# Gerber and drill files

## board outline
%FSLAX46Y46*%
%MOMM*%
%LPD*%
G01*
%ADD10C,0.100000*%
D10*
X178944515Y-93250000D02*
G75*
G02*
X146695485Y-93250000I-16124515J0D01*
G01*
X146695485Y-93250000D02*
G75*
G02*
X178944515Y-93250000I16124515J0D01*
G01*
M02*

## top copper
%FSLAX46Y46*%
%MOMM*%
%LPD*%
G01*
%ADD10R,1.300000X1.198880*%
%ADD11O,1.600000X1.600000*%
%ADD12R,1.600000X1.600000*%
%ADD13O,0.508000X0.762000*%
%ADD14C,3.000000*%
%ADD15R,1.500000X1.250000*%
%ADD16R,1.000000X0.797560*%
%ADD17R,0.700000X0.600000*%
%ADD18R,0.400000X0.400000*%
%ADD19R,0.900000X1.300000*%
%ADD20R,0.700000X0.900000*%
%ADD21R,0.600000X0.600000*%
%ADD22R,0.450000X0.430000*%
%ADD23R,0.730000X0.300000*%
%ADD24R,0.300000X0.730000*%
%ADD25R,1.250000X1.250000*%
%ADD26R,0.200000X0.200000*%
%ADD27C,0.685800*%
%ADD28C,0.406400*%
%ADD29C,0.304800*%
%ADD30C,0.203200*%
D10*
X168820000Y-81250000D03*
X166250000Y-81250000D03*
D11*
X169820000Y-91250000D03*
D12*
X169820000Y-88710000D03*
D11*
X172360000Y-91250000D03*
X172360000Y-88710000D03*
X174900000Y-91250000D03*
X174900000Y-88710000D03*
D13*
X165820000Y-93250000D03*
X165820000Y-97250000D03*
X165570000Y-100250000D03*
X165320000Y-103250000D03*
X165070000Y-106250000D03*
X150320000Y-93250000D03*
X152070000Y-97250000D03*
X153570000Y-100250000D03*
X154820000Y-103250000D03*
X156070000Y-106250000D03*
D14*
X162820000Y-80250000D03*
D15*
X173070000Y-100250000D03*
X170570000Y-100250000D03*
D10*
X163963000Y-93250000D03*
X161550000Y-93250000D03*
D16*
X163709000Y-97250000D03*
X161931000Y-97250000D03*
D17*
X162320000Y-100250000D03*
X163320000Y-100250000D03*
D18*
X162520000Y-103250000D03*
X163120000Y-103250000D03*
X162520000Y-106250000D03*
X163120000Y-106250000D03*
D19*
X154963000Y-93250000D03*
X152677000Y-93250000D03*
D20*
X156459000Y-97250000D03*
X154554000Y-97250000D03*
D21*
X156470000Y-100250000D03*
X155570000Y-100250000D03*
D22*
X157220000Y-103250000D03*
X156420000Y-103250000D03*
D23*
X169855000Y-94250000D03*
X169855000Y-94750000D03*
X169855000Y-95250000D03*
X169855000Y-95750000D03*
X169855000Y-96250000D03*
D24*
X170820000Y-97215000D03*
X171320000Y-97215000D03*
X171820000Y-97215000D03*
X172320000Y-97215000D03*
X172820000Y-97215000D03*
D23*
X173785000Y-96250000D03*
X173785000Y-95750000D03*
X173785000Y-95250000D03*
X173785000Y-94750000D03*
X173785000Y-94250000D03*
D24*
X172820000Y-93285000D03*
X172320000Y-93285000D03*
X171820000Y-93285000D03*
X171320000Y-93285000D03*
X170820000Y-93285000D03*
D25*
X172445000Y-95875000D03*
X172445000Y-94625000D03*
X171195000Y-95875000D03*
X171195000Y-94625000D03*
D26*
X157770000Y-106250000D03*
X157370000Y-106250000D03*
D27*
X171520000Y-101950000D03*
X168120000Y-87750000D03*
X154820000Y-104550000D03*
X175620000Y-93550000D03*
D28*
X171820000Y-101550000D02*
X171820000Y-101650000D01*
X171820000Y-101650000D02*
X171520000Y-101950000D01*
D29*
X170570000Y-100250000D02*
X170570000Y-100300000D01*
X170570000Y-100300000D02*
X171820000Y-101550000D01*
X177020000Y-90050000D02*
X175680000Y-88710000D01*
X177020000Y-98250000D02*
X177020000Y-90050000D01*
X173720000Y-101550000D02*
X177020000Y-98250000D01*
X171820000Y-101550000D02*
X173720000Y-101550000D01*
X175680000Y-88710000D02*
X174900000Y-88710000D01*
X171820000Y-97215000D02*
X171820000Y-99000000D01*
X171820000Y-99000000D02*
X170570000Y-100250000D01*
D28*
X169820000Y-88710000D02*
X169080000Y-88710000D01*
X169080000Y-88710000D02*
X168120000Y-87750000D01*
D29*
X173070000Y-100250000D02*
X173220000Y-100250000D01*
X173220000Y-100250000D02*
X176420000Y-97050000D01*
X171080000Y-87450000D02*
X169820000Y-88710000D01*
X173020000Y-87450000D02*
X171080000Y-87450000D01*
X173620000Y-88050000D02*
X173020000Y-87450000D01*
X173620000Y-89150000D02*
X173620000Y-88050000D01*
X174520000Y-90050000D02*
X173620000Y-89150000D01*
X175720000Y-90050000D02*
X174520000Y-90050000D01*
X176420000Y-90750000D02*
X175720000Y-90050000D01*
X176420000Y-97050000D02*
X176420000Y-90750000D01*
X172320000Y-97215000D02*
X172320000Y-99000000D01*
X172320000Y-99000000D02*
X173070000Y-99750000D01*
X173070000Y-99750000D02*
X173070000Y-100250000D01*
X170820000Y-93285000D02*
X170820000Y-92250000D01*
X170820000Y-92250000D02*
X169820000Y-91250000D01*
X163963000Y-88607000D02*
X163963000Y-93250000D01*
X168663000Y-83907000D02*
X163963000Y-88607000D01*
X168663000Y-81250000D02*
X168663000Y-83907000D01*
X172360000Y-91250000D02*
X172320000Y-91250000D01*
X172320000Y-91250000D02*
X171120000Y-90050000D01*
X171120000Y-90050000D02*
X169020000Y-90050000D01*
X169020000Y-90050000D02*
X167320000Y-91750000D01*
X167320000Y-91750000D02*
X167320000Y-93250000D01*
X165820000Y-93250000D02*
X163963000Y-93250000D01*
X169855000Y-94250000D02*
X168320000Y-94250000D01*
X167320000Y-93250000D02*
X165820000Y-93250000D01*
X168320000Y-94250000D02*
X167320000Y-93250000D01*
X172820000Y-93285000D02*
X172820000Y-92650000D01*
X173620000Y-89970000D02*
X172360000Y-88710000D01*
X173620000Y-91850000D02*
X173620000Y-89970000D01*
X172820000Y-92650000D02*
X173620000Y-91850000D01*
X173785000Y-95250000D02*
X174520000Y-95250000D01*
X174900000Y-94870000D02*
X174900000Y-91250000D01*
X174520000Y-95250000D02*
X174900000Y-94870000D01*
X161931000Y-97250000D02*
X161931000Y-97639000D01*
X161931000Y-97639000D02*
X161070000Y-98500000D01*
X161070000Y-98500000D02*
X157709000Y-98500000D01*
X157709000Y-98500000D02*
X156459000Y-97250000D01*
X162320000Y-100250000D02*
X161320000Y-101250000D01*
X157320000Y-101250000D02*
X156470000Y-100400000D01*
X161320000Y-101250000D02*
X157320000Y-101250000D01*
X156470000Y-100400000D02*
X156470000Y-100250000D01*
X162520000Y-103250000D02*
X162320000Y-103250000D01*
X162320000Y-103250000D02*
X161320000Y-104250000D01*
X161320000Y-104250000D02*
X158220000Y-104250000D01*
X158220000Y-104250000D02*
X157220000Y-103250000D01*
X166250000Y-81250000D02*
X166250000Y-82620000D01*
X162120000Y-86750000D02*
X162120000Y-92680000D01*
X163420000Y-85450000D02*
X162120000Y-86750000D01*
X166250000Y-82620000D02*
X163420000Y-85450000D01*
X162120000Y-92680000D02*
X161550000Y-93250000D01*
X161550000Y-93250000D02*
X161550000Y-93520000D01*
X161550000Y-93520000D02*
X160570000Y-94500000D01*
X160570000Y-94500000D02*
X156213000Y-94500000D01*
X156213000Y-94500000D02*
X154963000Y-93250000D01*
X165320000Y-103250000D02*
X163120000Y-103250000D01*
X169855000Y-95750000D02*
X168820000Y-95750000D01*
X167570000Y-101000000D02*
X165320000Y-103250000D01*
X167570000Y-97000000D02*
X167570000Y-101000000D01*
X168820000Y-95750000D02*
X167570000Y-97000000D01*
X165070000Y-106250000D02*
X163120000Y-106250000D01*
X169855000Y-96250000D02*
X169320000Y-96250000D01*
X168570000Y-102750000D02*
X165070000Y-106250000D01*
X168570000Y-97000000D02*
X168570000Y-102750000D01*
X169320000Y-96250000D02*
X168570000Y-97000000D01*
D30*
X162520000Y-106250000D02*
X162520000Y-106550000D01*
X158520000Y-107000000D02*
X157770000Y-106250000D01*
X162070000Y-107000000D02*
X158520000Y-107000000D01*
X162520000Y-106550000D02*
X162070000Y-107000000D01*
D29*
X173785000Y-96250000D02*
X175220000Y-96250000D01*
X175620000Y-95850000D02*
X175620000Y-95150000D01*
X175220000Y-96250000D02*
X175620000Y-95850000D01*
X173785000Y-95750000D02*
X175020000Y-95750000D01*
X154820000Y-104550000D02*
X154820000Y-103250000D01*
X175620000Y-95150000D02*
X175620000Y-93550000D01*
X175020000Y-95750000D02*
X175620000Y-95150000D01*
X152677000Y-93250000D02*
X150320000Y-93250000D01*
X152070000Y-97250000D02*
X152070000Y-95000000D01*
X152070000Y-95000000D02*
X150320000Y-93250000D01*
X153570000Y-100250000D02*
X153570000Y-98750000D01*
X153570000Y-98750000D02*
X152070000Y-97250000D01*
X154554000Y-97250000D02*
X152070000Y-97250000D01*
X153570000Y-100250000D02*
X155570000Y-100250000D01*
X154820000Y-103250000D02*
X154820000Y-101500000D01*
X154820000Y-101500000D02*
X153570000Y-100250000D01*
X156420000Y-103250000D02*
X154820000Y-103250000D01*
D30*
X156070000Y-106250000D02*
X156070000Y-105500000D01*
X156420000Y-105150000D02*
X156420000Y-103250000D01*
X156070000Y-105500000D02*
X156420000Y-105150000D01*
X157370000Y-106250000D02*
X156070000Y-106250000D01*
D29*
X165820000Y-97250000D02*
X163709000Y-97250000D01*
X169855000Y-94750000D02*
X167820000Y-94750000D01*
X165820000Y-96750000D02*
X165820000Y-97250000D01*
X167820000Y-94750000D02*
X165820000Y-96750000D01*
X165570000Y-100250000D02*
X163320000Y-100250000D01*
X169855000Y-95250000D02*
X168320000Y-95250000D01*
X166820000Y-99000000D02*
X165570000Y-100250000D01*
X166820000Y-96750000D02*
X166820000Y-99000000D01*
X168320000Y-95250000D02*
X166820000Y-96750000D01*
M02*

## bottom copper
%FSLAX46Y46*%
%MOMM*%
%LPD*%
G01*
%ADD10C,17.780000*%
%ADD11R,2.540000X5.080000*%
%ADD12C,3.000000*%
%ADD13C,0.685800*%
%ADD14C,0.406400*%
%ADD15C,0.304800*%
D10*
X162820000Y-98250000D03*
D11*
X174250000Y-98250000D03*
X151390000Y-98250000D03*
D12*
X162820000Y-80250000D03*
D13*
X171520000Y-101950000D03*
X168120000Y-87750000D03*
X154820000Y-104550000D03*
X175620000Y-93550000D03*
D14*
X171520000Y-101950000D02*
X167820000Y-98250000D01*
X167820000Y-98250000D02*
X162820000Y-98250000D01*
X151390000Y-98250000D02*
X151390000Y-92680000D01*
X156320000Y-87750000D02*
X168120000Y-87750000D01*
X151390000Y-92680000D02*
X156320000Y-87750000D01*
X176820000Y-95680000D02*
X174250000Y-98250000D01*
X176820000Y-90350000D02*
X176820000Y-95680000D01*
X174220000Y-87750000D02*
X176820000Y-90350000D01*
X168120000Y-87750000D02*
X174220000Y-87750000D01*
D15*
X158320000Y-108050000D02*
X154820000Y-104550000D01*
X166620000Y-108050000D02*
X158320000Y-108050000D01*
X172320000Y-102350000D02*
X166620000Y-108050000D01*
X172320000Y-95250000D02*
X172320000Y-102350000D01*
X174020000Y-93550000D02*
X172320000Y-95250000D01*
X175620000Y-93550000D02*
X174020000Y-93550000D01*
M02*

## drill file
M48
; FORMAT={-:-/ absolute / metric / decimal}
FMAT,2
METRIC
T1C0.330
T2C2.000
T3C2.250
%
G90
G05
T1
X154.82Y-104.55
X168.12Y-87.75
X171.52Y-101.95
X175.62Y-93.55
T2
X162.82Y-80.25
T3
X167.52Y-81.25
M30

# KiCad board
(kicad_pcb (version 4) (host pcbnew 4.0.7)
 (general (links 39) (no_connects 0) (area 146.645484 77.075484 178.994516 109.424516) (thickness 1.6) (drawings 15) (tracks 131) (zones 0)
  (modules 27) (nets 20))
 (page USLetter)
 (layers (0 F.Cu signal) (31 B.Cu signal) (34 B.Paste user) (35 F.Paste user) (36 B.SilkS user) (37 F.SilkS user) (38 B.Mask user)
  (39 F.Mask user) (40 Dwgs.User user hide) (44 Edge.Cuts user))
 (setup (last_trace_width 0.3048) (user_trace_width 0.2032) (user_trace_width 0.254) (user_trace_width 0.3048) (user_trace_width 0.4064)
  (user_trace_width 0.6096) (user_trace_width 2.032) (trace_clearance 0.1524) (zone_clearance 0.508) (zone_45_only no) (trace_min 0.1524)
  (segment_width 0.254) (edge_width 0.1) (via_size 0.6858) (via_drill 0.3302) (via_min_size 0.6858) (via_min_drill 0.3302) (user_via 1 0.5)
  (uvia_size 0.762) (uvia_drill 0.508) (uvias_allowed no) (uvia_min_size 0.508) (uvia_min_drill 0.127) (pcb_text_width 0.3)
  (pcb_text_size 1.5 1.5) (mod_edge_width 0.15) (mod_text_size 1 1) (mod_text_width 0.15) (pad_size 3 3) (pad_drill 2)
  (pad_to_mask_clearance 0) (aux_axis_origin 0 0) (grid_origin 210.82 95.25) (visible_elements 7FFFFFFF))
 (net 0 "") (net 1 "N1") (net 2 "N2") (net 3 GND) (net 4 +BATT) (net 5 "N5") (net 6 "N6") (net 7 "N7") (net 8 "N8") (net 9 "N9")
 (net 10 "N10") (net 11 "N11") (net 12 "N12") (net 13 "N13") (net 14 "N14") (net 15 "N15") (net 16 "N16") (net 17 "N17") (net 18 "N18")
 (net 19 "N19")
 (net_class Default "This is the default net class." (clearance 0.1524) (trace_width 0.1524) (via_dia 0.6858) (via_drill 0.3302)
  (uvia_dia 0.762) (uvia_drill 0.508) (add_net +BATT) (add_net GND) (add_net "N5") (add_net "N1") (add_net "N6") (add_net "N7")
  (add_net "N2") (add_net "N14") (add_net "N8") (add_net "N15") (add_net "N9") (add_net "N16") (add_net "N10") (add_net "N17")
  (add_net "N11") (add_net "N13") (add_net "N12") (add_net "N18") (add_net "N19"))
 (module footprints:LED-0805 (layer F.Cu) (at 167.52 81.25)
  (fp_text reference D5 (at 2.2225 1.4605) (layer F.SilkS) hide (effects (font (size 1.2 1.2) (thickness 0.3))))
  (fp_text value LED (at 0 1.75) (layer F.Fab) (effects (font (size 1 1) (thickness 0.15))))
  (pad 2 smd rect (at 1.3 0 180) (size 1.3 1.19888) (layers F.Cu F.Paste F.Mask) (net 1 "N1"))
  (pad 1 smd rect (at -1.27 0 180) (size 1.3 1.19888) (layers F.Cu F.Paste F.Mask) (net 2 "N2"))
  (pad "" np_thru_hole circle (at 0 0) (size 2.25 2.25) (drill 2.25) (layers *.Cu *.Mask)))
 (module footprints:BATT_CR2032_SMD (layer B.Cu) (at 162.82 98.25 180)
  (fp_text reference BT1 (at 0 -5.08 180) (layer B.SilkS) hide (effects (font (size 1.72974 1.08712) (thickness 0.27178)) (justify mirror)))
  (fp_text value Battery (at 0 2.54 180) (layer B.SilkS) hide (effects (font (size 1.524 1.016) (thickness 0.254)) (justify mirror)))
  (pad 2 smd circle (at 0 0 180) (size 17.78 17.78) (layers B.Cu B.Paste B.Mask) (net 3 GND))
  (pad 1 smd rect (at -11.43 0 180) (size 2.54 5.08) (layers B.Cu B.Paste B.Mask) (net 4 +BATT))
  (pad 1 smd rect (at 11.43 0 180) (size 2.54 5.08) (layers B.Cu B.Paste B.Mask) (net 4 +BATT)))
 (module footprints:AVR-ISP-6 (layer F.Cu) (at 169.82 91.25 90)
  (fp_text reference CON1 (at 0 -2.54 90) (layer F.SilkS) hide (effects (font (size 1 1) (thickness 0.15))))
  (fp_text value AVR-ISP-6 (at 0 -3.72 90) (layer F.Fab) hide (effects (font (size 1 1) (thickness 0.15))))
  (pad 1 smd oval (at 0 0 90) (size 1.6 1.6) (layers F.Cu F.Paste F.Mask) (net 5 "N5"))
  (pad 2 smd rect (at 2.54 0 90) (size 1.6 1.6) (layers F.Cu F.Paste F.Mask) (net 4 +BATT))
  (pad 3 smd oval (at 0 2.54 90) (size 1.6 1.6) (layers F.Cu F.Paste F.Mask) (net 1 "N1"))
  (pad 4 smd oval (at 2.54 2.54 90) (size 1.6 1.6) (layers F.Cu F.Paste F.Mask) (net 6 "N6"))
  (pad 5 smd oval (at 0 5.08 90) (size 1.6 1.6) (layers F.Cu F.Paste F.Mask) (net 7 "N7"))
  (pad 6 smd oval (at 2.54 5.08 90) (size 1.6 1.6) (layers F.Cu F.Paste F.Mask) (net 3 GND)))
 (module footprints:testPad (layer F.Cu) (at 165.82 93.25)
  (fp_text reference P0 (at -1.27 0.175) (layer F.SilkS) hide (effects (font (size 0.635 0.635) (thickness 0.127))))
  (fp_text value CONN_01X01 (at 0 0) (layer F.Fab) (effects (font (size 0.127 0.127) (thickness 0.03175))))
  (pad 1 smd oval (at 0 0) (size 0.508 0.762) (layers F.Cu F.Paste F.Mask) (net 1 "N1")))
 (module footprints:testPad (layer F.Cu) (at 165.82 97.25)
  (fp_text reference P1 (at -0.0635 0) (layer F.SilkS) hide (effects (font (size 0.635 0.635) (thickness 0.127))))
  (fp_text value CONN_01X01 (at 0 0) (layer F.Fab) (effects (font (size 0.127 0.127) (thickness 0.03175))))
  (pad 1 smd oval (at 0 0) (size 0.508 0.762) (layers F.Cu F.Paste F.Mask) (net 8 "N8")))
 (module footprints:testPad (layer F.Cu) (at 165.57 100.25)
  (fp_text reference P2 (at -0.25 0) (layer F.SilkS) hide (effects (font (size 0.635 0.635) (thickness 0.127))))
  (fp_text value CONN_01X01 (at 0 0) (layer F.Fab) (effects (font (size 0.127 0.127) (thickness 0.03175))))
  (pad 1 smd oval (at 0 0) (size 0.508 0.762) (layers F.Cu F.Paste F.Mask) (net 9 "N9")))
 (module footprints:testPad (layer F.Cu) (at 165.32 103.25)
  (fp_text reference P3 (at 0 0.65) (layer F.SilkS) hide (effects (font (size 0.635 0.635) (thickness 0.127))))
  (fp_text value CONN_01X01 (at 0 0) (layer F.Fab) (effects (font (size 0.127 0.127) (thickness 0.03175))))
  (pad 1 smd oval (at 0 0) (size 0.508 0.762) (layers F.Cu F.Paste F.Mask) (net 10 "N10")))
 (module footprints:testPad (layer F.Cu) (at 165.07 106.25)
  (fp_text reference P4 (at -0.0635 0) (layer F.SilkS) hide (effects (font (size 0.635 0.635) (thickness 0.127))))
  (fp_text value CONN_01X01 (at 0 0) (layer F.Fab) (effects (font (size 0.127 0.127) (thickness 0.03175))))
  (pad 1 smd oval (at 0 0) (size 0.508 0.762) (layers F.Cu F.Paste F.Mask) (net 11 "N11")))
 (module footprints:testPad (layer F.Cu) (at 150.32 93.25)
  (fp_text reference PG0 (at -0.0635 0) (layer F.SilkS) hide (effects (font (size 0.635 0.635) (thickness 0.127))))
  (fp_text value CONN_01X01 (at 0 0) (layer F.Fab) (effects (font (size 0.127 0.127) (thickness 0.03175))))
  (pad 1 smd oval (at 0 0) (size 0.508 0.762) (layers F.Cu F.Paste F.Mask) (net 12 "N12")))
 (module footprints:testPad (layer F.Cu) (at 152.07 97.25)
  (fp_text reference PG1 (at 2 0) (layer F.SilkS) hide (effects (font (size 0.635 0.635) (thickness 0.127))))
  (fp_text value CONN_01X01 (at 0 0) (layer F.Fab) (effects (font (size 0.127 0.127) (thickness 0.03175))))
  (pad 1 smd oval (at 0 0) (size 0.508 0.762) (layers F.Cu F.Paste F.Mask) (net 12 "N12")))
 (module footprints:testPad (layer F.Cu) (at 153.57 100.25)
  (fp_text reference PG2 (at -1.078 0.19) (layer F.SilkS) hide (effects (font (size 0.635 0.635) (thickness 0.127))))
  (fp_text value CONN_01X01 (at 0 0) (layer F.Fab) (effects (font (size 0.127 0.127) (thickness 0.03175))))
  (pad 1 smd oval (at 0 0) (size 0.508 0.762) (layers F.Cu F.Paste F.Mask) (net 12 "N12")))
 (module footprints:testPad (layer F.Cu) (at 154.82 103.25)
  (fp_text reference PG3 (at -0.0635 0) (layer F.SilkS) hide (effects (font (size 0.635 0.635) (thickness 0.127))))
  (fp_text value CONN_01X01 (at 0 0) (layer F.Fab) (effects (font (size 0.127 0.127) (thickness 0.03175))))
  (pad 1 smd oval (at 0 0) (size 0.508 0.762) (layers F.Cu F.Paste F.Mask) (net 12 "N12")))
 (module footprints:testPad (layer F.Cu) (at 156.07 106.25)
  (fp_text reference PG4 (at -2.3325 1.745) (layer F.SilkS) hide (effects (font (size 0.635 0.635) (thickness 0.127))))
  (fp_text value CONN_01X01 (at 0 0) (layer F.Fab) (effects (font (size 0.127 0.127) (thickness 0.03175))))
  (pad 1 smd oval (at 0 0) (size 0.508 0.762) (layers F.Cu F.Paste F.Mask) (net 12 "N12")))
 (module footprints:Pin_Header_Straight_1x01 (layer F.Cu) (at 162.82 80.25)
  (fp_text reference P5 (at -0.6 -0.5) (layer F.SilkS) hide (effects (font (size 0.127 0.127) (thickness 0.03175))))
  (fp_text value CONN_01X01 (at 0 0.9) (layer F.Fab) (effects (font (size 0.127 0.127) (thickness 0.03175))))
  (pad 1 thru_hole circle (at 0 0) (size 3 3) (drill 2) (layers *.Cu *.Mask) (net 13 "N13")))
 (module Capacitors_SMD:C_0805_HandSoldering (layer F.Cu) (at 171.82 100.25 180)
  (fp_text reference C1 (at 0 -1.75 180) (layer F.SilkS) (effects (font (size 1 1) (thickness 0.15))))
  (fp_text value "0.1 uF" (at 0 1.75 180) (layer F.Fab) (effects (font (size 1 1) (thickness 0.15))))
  (pad 1 smd rect (at -1.25 0 180) (size 1.5 1.25) (layers F.Cu F.Paste F.Mask) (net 4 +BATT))
  (pad 2 smd rect (at 1.25 0 180) (size 1.5 1.25) (layers F.Cu F.Paste F.Mask) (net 3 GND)))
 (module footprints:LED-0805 (layer F.Cu) (at 162.82 93.25)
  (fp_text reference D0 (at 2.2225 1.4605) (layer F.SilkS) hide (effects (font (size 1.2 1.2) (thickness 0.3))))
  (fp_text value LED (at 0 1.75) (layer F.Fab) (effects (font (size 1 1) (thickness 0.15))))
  (pad 2 smd rect (at 1.143 0 180) (size 1.3 1.19888) (layers F.Cu F.Paste F.Mask) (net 1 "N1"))
  (pad 1 smd rect (at -1.27 0 180) (size 1.3 1.19888) (layers F.Cu F.Paste F.Mask) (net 2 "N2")))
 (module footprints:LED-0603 (layer F.Cu) (at 162.82 97.25)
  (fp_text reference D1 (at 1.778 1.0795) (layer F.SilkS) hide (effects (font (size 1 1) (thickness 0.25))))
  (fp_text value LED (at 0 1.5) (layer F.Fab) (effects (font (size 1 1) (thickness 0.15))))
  (pad 2 smd rect (at 0.889 0 180) (size 1 0.79756) (layers F.Cu F.Paste F.Mask) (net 8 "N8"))
  (pad 1 smd rect (at -0.889 0 180) (size 1 0.79756) (layers F.Cu F.Paste F.Mask) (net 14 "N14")))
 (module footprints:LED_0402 (layer F.Cu) (at 162.82 100.25)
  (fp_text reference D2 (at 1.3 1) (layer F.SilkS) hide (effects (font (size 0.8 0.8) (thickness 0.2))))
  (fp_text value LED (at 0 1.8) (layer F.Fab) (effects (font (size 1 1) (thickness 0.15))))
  (pad 1 smd rect (at -0.5 0) (size 0.7 0.6) (layers F.Cu F.Paste F.Mask) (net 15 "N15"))
  (pad 2 smd rect (at 0.5 0) (size 0.7 0.6) (layers F.Cu F.Paste F.Mask) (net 9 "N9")))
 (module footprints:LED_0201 (layer F.Cu) (at 162.82 103.25)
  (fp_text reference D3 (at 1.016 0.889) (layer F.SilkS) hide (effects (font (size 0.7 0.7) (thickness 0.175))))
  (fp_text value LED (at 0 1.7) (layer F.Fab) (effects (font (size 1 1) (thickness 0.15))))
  (pad 1 smd rect (at -0.3 0) (size 0.4 0.4) (layers F.Cu F.Paste F.Mask) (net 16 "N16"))
  (pad 2 smd rect (at 0.3 0) (size 0.4 0.4) (layers F.Cu F.Paste F.Mask) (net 10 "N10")))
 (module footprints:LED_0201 (layer F.Cu) (at 162.82 106.25)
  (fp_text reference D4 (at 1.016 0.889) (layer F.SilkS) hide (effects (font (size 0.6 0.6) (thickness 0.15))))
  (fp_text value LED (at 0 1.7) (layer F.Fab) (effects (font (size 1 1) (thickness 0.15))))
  (pad 1 smd rect (at -0.3 0) (size 0.4 0.4) (layers F.Cu F.Paste F.Mask) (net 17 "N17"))
  (pad 2 smd rect (at 0.3 0) (size 0.4 0.4) (layers F.Cu F.Paste F.Mask) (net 11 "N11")))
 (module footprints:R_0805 (layer F.Cu) (at 153.82 93.25 180)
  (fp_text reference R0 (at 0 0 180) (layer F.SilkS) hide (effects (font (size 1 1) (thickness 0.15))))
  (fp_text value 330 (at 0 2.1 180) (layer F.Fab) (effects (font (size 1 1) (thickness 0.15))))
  (pad 1 smd rect (at -1.143 0 180) (size 0.9 1.3) (layers F.Cu F.Paste F.Mask) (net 2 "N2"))
  (pad 2 smd rect (at 1.143 0 180) (size 0.9 1.3) (layers F.Cu F.Paste F.Mask) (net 12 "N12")))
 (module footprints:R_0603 (layer F.Cu) (at 155.57 97.25 180)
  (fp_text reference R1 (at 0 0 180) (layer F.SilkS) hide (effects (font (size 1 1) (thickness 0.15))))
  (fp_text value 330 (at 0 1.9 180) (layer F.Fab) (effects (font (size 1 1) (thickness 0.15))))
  (pad 1 smd rect (at -0.889 0 180) (size 0.7 0.9) (layers F.Cu F.Paste F.Mask) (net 14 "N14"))
  (pad 2 smd rect (at 1.016 0 180) (size 0.7 0.9) (layers F.Cu F.Paste F.Mask) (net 12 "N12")))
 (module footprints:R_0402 (layer F.Cu) (at 156.07 100.25 180)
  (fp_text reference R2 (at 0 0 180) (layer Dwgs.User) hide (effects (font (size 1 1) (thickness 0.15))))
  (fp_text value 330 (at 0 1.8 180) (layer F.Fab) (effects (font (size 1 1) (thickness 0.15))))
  (pad 1 smd rect (at -0.4 0 180) (size 0.6 0.6) (layers F.Cu F.Paste F.Mask) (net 15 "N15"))
  (pad 2 smd rect (at 0.5 0 180) (size 0.6 0.6) (layers F.Cu F.Paste F.Mask) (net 12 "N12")))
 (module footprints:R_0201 (layer F.Cu) (at 156.82 103.25 180)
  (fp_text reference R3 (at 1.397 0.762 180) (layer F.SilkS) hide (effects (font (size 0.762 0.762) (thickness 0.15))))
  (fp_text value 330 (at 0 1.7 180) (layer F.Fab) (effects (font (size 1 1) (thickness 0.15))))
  (pad 1 smd rect (at -0.4 0 180) (size 0.45 0.43) (layers F.Cu F.Paste F.Mask) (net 16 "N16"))
  (pad 2 smd rect (at 0.4 0 180) (size 0.45 0.43) (layers F.Cu F.Paste F.Mask) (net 12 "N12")))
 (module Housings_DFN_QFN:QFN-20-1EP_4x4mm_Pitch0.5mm (layer F.Cu) (at 171.82 95.25)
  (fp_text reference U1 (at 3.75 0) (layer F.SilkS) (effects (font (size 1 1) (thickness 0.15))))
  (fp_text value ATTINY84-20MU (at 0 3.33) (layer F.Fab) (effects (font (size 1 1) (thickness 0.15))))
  (pad 1 smd rect (at -1.965 -1) (size 0.73 0.3) (layers F.Cu F.Paste F.Mask) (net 1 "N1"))
  (pad 2 smd rect (at -1.965 -0.5) (size 0.73 0.3) (layers F.Cu F.Paste F.Mask) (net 8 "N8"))
  (pad 3 smd rect (at -1.965 0) (size 0.73 0.3) (layers F.Cu F.Paste F.Mask) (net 9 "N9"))
  (pad 4 smd rect (at -1.965 0.5) (size 0.73 0.3) (layers F.Cu F.Paste F.Mask) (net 10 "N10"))
  (pad 5 smd rect (at -1.965 1) (size 0.73 0.3) (layers F.Cu F.Paste F.Mask) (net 11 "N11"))
  (pad 6 smd rect (at -1 1.965 90) (size 0.73 0.3) (layers F.Cu F.Paste F.Mask))
  (pad 7 smd rect (at -0.5 1.965 90) (size 0.73 0.3) (layers F.Cu F.Paste F.Mask))
  (pad 8 smd rect (at 0 1.965 90) (size 0.73 0.3) (layers F.Cu F.Paste F.Mask) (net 3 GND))
  (pad 9 smd rect (at 0.5 1.965 90) (size 0.73 0.3) (layers F.Cu F.Paste F.Mask) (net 4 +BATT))
  (pad 10 smd rect (at 1 1.965 90) (size 0.73 0.3) (layers F.Cu F.Paste F.Mask))
  (pad 11 smd rect (at 1.965 1) (size 0.73 0.3) (layers F.Cu F.Paste F.Mask) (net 12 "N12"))
  (pad 12 smd rect (at 1.965 0.5) (size 0.73 0.3) (layers F.Cu F.Paste F.Mask) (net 12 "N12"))
  (pad 13 smd rect (at 1.965 0) (size 0.73 0.3) (layers F.Cu F.Paste F.Mask) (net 7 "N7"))
  (pad 14 smd rect (at 1.965 -0.5) (size 0.73 0.3) (layers F.Cu F.Paste F.Mask) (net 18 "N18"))
  (pad 15 smd rect (at 1.965 -1) (size 0.73 0.3) (layers F.Cu F.Paste F.Mask) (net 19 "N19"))
  (pad 16 smd rect (at 1 -1.965 90) (size 0.73 0.3) (layers F.Cu F.Paste F.Mask) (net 6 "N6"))
  (pad 17 smd rect (at 0.5 -1.965 90) (size 0.73 0.3) (layers F.Cu F.Paste F.Mask))
  (pad 18 smd rect (at 0 -1.965 90) (size 0.73 0.3) (layers F.Cu F.Paste F.Mask))
  (pad 19 smd rect (at -0.5 -1.965 90) (size 0.73 0.3) (layers F.Cu F.Paste F.Mask))
  (pad 20 smd rect (at -1 -1.965 90) (size 0.73 0.3) (layers F.Cu F.Paste F.Mask) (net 5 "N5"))
  (pad 21 smd rect (at 0.625 0.625) (size 1.25 1.25) (layers F.Cu F.Paste F.Mask) (solder_paste_margin_ratio -0.2))
  (pad 21 smd rect (at 0.625 -0.625) (size 1.25 1.25) (layers F.Cu F.Paste F.Mask) (solder_paste_margin_ratio -0.2))
  (pad 21 smd rect (at -0.625 0.625) (size 1.25 1.25) (layers F.Cu F.Paste F.Mask) (solder_paste_margin_ratio -0.2))
  (pad 21 smd rect (at -0.625 -0.625) (size 1.25 1.25) (layers F.Cu F.Paste F.Mask) (solder_paste_margin_ratio -0.2)))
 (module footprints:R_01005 (layer F.Cu) (at 157.57 106.25 180)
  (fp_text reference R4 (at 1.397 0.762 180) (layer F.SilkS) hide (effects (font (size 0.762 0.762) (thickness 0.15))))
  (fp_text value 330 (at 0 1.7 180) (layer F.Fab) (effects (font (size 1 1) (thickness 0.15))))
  (pad 1 smd rect (at -0.2 0 180) (size 0.2 0.2) (layers F.Cu F.Paste F.Mask) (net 17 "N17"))
  (pad 2 smd rect (at 0.2 0 180) (size 0.2 0.2) (layers F.Cu F.Paste F.Mask) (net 12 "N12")))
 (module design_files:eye (layer F.Cu) (at 167.42 81.05)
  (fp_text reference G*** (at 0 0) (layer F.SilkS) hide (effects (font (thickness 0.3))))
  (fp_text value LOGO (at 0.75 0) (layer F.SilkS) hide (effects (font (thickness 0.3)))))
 (gr_circle (center 162.82 93.25) (end 148.82 85.25) (layer Edge.Cuts) (width 0.1))
 (segment (start 171.82 101.55) (end 171.82 101.65) (width 0.4064) (layer F.Cu) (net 3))
 (segment (start 171.52 101.95) (end 167.82 98.25) (width 0.4064) (layer B.Cu) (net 3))
 (via (at 171.52 101.95) (size 0.6858) (drill 0.3302) (layers F.Cu B.Cu) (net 3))
 (segment (start 171.82 101.65) (end 171.52 101.95) (width 0.4064) (layer F.Cu) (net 3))
 (segment (start 167.82 98.25) (end 162.82 98.25) (width 0.4064) (layer B.Cu) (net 3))
 (segment (start 170.57 100.25) (end 170.57 100.3) (width 0.3048) (layer F.Cu) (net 3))
 (segment (start 170.57 100.3) (end 171.82 101.55) (width 0.3048) (layer F.Cu) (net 3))
 (segment (start 177.02 90.05) (end 175.68 88.71) (width 0.3048) (layer F.Cu) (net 3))
 (segment (start 177.02 98.25) (end 177.02 90.05) (width 0.3048) (layer F.Cu) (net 3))
 (segment (start 173.72 101.55) (end 177.02 98.25) (width 0.3048) (layer F.Cu) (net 3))
 (segment (start 171.82 101.55) (end 173.72 101.55) (width 0.3048) (layer F.Cu) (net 3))
 (segment (start 175.68 88.71) (end 174.9 88.71) (width 0.3048) (layer F.Cu) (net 3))
 (segment (start 171.82 97.215) (end 171.82 99) (width 0.3048) (layer F.Cu) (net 3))
 (segment (start 171.82 99) (end 170.57 100.25) (width 0.3048) (layer F.Cu) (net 3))
 (segment (start 151.39 98.25) (end 151.39 92.68) (width 0.4064) (layer B.Cu) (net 4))
 (segment (start 156.32 87.75) (end 168.12 87.75) (width 0.4064) (layer B.Cu) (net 4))
 (segment (start 151.39 92.68) (end 156.32 87.75) (width 0.4064) (layer B.Cu) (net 4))
 (segment (start 169.82 88.71) (end 169.08 88.71) (width 0.4064) (layer F.Cu) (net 4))
 (segment (start 169.08 88.71) (end 168.12 87.75) (width 0.4064) (layer F.Cu) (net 4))
 (segment (start 176.82 95.68) (end 174.25 98.25) (width 0.4064) (layer B.Cu) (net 4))
 (segment (start 176.82 90.35) (end 176.82 95.68) (width 0.4064) (layer B.Cu) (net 4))
 (segment (start 174.22 87.75) (end 176.82 90.35) (width 0.4064) (layer B.Cu) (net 4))
 (segment (start 168.12 87.75) (end 174.22 87.75) (width 0.4064) (layer B.Cu) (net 4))
 (via (at 168.12 87.75) (size 0.6858) (drill 0.3302) (layers F.Cu B.Cu) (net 4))
 (segment (start 173.07 100.25) (end 173.22 100.25) (width 0.3048) (layer F.Cu) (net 4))
 (segment (start 173.22 100.25) (end 176.42 97.05) (width 0.3048) (layer F.Cu) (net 4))
 (segment (start 171.08 87.45) (end 169.82 88.71) (width 0.3048) (layer F.Cu) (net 4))
 (segment (start 173.02 87.45) (end 171.08 87.45) (width 0.3048) (layer F.Cu) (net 4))
 (segment (start 173.62 88.05) (end 173.02 87.45) (width 0.3048) (layer F.Cu) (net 4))
 (segment (start 173.62 89.15) (end 173.62 88.05) (width 0.3048) (layer F.Cu) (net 4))
 (segment (start 174.52 90.05) (end 173.62 89.15) (width 0.3048) (layer F.Cu) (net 4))
 (segment (start 175.72 90.05) (end 174.52 90.05) (width 0.3048) (layer F.Cu) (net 4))
 (segment (start 176.42 90.75) (end 175.72 90.05) (width 0.3048) (layer F.Cu) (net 4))
 (segment (start 176.42 97.05) (end 176.42 90.75) (width 0.3048) (layer F.Cu) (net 4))
 (segment (start 172.32 97.215) (end 172.32 99) (width 0.3048) (layer F.Cu) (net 4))
 (segment (start 172.32 99) (end 173.07 99.75) (width 0.3048) (layer F.Cu) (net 4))
 (segment (start 173.07 99.75) (end 173.07 100.25) (width 0.3048) (layer F.Cu) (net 4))
 (segment (start 170.82 93.285) (end 170.82 92.25) (width 0.3048) (layer F.Cu) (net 5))
 (segment (start 170.82 92.25) (end 169.82 91.25) (width 0.3048) (layer F.Cu) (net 5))
 (segment (start 163.963 88.607) (end 163.963 93.25) (width 0.3048) (layer F.Cu) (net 1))
 (segment (start 168.663 83.907) (end 163.963 88.607) (width 0.3048) (layer F.Cu) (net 1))
 (segment (start 168.663 81.25) (end 168.663 83.907) (width 0.3048) (layer F.Cu) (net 1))
 (segment (start 172.36 91.25) (end 172.32 91.25) (width 0.3048) (layer F.Cu) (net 1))
 (segment (start 172.32 91.25) (end 171.12 90.05) (width 0.3048) (layer F.Cu) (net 1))
 (segment (start 171.12 90.05) (end 169.02 90.05) (width 0.3048) (layer F.Cu) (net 1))
 (segment (start 169.02 90.05) (end 167.32 91.75) (width 0.3048) (layer F.Cu) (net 1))
 (segment (start 167.32 91.75) (end 167.32 93.25) (width 0.3048) (layer F.Cu) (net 1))
 (segment (start 165.82 93.25) (end 163.963 93.25) (width 0.3048) (layer F.Cu) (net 1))
 (segment (start 169.855 94.25) (end 168.32 94.25) (width 0.3048) (layer F.Cu) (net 1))
 (segment (start 167.32 93.25) (end 165.82 93.25) (width 0.3048) (layer F.Cu) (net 1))
 (segment (start 168.32 94.25) (end 167.32 93.25) (width 0.3048) (layer F.Cu) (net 1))
 (segment (start 172.82 93.285) (end 172.82 92.65) (width 0.3048) (layer F.Cu) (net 6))
 (segment (start 173.62 89.97) (end 172.36 88.71) (width 0.3048) (layer F.Cu) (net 6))
 (segment (start 173.62 91.85) (end 173.62 89.97) (width 0.3048) (layer F.Cu) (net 6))
 (segment (start 172.82 92.65) (end 173.62 91.85) (width 0.3048) (layer F.Cu) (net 6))
 (segment (start 173.785 95.25) (end 174.52 95.25) (width 0.3048) (layer F.Cu) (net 7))
 (segment (start 174.9 94.87) (end 174.9 91.25) (width 0.3048) (layer F.Cu) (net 7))
 (segment (start 174.52 95.25) (end 174.9 94.87) (width 0.3048) (layer F.Cu) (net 7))
 (segment (start 161.931 97.25) (end 161.931 97.639) (width 0.3048) (layer F.Cu) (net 14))
 (segment (start 161.931 97.639) (end 161.07 98.5) (width 0.3048) (layer F.Cu) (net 14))
 (segment (start 161.07 98.5) (end 157.709 98.5) (width 0.3048) (layer F.Cu) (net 14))
 (segment (start 157.709 98.5) (end 156.459 97.25) (width 0.3048) (layer F.Cu) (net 14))
 (segment (start 162.32 100.25) (end 161.32 101.25) (width 0.3048) (layer F.Cu) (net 15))
 (segment (start 157.32 101.25) (end 156.47 100.4) (width 0.3048) (layer F.Cu) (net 15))
 (segment (start 161.32 101.25) (end 157.32 101.25) (width 0.3048) (layer F.Cu) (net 15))
 (segment (start 156.47 100.4) (end 156.47 100.25) (width 0.3048) (layer F.Cu) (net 15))
 (segment (start 162.52 103.25) (end 162.32 103.25) (width 0.3048) (layer F.Cu) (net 16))
 (segment (start 162.32 103.25) (end 161.32 104.25) (width 0.3048) (layer F.Cu) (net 16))
 (segment (start 161.32 104.25) (end 158.22 104.25) (width 0.3048) (layer F.Cu) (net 16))
 (segment (start 158.22 104.25) (end 157.22 103.25) (width 0.3048) (layer F.Cu) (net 16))
 (segment (start 166.25 81.25) (end 166.25 82.62) (width 0.3048) (layer F.Cu) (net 2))
 (segment (start 162.12 86.75) (end 162.12 92.68) (width 0.3048) (layer F.Cu) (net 2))
 (segment (start 163.42 85.45) (end 162.12 86.75) (width 0.3048) (layer F.Cu) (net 2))
 (segment (start 166.25 82.62) (end 163.42 85.45) (width 0.3048) (layer F.Cu) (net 2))
 (segment (start 162.12 92.68) (end 161.55 93.25) (width 0.3048) (layer F.Cu) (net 2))
 (segment (start 161.55 93.25) (end 161.55 93.52) (width 0.3048) (layer F.Cu) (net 2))
 (segment (start 161.55 93.52) (end 160.57 94.5) (width 0.3048) (layer F.Cu) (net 2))
 (segment (start 160.57 94.5) (end 156.213 94.5) (width 0.3048) (layer F.Cu) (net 2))
 (segment (start 156.213 94.5) (end 154.963 93.25) (width 0.3048) (layer F.Cu) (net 2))
 (segment (start 165.32 103.25) (end 163.12 103.25) (width 0.3048) (layer F.Cu) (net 10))
 (segment (start 169.855 95.75) (end 168.82 95.75) (width 0.3048) (layer F.Cu) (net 10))
 (segment (start 167.57 101) (end 165.32 103.25) (width 0.3048) (layer F.Cu) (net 10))
 (segment (start 167.57 97) (end 167.57 101) (width 0.3048) (layer F.Cu) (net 10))
 (segment (start 168.82 95.75) (end 167.57 97) (width 0.3048) (layer F.Cu) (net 10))
 (segment (start 165.07 106.25) (end 163.12 106.25) (width 0.3048) (layer F.Cu) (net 11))
 (segment (start 169.855 96.25) (end 169.32 96.25) (width 0.3048) (layer F.Cu) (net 11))
 (segment (start 168.57 102.75) (end 165.07 106.25) (width 0.3048) (layer F.Cu) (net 11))
 (segment (start 168.57 97) (end 168.57 102.75) (width 0.3048) (layer F.Cu) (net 11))
 (segment (start 169.32 96.25) (end 168.57 97) (width 0.3048) (layer F.Cu) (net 11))
 (segment (start 162.52 106.25) (end 162.52 106.55) (width 0.2032) (layer F.Cu) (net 17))
 (segment (start 158.52 107) (end 157.77 106.25) (width 0.2032) (layer F.Cu) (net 17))
 (segment (start 162.07 107) (end 158.52 107) (width 0.2032) (layer F.Cu) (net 17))
 (segment (start 162.52 106.55) (end 162.07 107) (width 0.2032) (layer F.Cu) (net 17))
 (segment (start 173.785 96.25) (end 175.22 96.25) (width 0.3048) (layer F.Cu) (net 12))
 (segment (start 175.62 95.85) (end 175.62 95.15) (width 0.3048) (layer F.Cu) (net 12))
 (segment (start 175.22 96.25) (end 175.62 95.85) (width 0.3048) (layer F.Cu) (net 12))
 (segment (start 173.785 95.75) (end 175.02 95.75) (width 0.3048) (layer F.Cu) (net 12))
 (segment (start 154.82 104.55) (end 154.82 103.25) (width 0.3048) (layer F.Cu) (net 12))
 (via (at 154.82 104.55) (size 0.6858) (drill 0.3302) (layers F.Cu B.Cu) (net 12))
 (segment (start 158.32 108.05) (end 154.82 104.55) (width 0.3048) (layer B.Cu) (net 12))
 (segment (start 166.62 108.05) (end 158.32 108.05) (width 0.3048) (layer B.Cu) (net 12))
 (segment (start 172.32 102.35) (end 166.62 108.05) (width 0.3048) (layer B.Cu) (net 12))
 (segment (start 172.32 95.25) (end 172.32 102.35) (width 0.3048) (layer B.Cu) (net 12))
 (segment (start 174.02 93.55) (end 172.32 95.25) (width 0.3048) (layer B.Cu) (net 12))
 (segment (start 175.62 93.55) (end 174.02 93.55) (width 0.3048) (layer B.Cu) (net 12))
 (via (at 175.62 93.55) (size 0.6858) (drill 0.3302) (layers F.Cu B.Cu) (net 12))
 (segment (start 175.62 95.15) (end 175.62 93.55) (width 0.3048) (layer F.Cu) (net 12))
 (segment (start 175.02 95.75) (end 175.62 95.15) (width 0.3048) (layer F.Cu) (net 12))
 (segment (start 152.677 93.25) (end 150.32 93.25) (width 0.3048) (layer F.Cu) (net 12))
 (segment (start 152.07 97.25) (end 152.07 95) (width 0.3048) (layer F.Cu) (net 12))
 (segment (start 152.07 95) (end 150.32 93.25) (width 0.3048) (layer F.Cu) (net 12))
 (segment (start 153.57 100.25) (end 153.57 98.75) (width 0.3048) (layer F.Cu) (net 12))
 (segment (start 153.57 98.75) (end 152.07 97.25) (width 0.3048) (layer F.Cu) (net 12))
 (segment (start 154.554 97.25) (end 152.07 97.25) (width 0.3048) (layer F.Cu) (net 12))
 (segment (start 153.57 100.25) (end 155.57 100.25) (width 0.3048) (layer F.Cu) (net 12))
 (segment (start 154.82 103.25) (end 154.82 101.5) (width 0.3048) (layer F.Cu) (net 12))
 (segment (start 154.82 101.5) (end 153.57 100.25) (width 0.3048) (layer F.Cu) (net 12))
 (segment (start 156.42 103.25) (end 154.82 103.25) (width 0.3048) (layer F.Cu) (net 12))
 (segment (start 156.07 106.25) (end 156.07 105.5) (width 0.2032) (layer F.Cu) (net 12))
 (segment (start 156.42 105.15) (end 156.42 103.25) (width 0.2032) (layer F.Cu) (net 12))
 (segment (start 156.07 105.5) (end 156.42 105.15) (width 0.2032) (layer F.Cu) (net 12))
 (segment (start 157.37 106.25) (end 156.07 106.25) (width 0.2032) (layer F.Cu) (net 12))
 (segment (start 165.82 97.25) (end 163.709 97.25) (width 0.3048) (layer F.Cu) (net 8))
 (segment (start 169.855 94.75) (end 167.82 94.75) (width 0.3048) (layer F.Cu) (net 8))
 (segment (start 165.82 96.75) (end 165.82 97.25) (width 0.3048) (layer F.Cu) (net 8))
 (segment (start 167.82 94.75) (end 165.82 96.75) (width 0.3048) (layer F.Cu) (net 8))
 (segment (start 165.57 100.25) (end 163.32 100.25) (width 0.3048) (layer F.Cu) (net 9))
 (segment (start 169.855 95.25) (end 168.32 95.25) (width 0.3048) (layer F.Cu) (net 9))
 (segment (start 166.82 99) (end 165.57 100.25) (width 0.3048) (layer F.Cu) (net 9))
 (segment (start 166.82 96.75) (end 166.82 99) (width 0.3048) (layer F.Cu) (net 9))
 (segment (start 168.32 95.25) (end 166.82 96.75) (width 0.3048) (layer F.Cu) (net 9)))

